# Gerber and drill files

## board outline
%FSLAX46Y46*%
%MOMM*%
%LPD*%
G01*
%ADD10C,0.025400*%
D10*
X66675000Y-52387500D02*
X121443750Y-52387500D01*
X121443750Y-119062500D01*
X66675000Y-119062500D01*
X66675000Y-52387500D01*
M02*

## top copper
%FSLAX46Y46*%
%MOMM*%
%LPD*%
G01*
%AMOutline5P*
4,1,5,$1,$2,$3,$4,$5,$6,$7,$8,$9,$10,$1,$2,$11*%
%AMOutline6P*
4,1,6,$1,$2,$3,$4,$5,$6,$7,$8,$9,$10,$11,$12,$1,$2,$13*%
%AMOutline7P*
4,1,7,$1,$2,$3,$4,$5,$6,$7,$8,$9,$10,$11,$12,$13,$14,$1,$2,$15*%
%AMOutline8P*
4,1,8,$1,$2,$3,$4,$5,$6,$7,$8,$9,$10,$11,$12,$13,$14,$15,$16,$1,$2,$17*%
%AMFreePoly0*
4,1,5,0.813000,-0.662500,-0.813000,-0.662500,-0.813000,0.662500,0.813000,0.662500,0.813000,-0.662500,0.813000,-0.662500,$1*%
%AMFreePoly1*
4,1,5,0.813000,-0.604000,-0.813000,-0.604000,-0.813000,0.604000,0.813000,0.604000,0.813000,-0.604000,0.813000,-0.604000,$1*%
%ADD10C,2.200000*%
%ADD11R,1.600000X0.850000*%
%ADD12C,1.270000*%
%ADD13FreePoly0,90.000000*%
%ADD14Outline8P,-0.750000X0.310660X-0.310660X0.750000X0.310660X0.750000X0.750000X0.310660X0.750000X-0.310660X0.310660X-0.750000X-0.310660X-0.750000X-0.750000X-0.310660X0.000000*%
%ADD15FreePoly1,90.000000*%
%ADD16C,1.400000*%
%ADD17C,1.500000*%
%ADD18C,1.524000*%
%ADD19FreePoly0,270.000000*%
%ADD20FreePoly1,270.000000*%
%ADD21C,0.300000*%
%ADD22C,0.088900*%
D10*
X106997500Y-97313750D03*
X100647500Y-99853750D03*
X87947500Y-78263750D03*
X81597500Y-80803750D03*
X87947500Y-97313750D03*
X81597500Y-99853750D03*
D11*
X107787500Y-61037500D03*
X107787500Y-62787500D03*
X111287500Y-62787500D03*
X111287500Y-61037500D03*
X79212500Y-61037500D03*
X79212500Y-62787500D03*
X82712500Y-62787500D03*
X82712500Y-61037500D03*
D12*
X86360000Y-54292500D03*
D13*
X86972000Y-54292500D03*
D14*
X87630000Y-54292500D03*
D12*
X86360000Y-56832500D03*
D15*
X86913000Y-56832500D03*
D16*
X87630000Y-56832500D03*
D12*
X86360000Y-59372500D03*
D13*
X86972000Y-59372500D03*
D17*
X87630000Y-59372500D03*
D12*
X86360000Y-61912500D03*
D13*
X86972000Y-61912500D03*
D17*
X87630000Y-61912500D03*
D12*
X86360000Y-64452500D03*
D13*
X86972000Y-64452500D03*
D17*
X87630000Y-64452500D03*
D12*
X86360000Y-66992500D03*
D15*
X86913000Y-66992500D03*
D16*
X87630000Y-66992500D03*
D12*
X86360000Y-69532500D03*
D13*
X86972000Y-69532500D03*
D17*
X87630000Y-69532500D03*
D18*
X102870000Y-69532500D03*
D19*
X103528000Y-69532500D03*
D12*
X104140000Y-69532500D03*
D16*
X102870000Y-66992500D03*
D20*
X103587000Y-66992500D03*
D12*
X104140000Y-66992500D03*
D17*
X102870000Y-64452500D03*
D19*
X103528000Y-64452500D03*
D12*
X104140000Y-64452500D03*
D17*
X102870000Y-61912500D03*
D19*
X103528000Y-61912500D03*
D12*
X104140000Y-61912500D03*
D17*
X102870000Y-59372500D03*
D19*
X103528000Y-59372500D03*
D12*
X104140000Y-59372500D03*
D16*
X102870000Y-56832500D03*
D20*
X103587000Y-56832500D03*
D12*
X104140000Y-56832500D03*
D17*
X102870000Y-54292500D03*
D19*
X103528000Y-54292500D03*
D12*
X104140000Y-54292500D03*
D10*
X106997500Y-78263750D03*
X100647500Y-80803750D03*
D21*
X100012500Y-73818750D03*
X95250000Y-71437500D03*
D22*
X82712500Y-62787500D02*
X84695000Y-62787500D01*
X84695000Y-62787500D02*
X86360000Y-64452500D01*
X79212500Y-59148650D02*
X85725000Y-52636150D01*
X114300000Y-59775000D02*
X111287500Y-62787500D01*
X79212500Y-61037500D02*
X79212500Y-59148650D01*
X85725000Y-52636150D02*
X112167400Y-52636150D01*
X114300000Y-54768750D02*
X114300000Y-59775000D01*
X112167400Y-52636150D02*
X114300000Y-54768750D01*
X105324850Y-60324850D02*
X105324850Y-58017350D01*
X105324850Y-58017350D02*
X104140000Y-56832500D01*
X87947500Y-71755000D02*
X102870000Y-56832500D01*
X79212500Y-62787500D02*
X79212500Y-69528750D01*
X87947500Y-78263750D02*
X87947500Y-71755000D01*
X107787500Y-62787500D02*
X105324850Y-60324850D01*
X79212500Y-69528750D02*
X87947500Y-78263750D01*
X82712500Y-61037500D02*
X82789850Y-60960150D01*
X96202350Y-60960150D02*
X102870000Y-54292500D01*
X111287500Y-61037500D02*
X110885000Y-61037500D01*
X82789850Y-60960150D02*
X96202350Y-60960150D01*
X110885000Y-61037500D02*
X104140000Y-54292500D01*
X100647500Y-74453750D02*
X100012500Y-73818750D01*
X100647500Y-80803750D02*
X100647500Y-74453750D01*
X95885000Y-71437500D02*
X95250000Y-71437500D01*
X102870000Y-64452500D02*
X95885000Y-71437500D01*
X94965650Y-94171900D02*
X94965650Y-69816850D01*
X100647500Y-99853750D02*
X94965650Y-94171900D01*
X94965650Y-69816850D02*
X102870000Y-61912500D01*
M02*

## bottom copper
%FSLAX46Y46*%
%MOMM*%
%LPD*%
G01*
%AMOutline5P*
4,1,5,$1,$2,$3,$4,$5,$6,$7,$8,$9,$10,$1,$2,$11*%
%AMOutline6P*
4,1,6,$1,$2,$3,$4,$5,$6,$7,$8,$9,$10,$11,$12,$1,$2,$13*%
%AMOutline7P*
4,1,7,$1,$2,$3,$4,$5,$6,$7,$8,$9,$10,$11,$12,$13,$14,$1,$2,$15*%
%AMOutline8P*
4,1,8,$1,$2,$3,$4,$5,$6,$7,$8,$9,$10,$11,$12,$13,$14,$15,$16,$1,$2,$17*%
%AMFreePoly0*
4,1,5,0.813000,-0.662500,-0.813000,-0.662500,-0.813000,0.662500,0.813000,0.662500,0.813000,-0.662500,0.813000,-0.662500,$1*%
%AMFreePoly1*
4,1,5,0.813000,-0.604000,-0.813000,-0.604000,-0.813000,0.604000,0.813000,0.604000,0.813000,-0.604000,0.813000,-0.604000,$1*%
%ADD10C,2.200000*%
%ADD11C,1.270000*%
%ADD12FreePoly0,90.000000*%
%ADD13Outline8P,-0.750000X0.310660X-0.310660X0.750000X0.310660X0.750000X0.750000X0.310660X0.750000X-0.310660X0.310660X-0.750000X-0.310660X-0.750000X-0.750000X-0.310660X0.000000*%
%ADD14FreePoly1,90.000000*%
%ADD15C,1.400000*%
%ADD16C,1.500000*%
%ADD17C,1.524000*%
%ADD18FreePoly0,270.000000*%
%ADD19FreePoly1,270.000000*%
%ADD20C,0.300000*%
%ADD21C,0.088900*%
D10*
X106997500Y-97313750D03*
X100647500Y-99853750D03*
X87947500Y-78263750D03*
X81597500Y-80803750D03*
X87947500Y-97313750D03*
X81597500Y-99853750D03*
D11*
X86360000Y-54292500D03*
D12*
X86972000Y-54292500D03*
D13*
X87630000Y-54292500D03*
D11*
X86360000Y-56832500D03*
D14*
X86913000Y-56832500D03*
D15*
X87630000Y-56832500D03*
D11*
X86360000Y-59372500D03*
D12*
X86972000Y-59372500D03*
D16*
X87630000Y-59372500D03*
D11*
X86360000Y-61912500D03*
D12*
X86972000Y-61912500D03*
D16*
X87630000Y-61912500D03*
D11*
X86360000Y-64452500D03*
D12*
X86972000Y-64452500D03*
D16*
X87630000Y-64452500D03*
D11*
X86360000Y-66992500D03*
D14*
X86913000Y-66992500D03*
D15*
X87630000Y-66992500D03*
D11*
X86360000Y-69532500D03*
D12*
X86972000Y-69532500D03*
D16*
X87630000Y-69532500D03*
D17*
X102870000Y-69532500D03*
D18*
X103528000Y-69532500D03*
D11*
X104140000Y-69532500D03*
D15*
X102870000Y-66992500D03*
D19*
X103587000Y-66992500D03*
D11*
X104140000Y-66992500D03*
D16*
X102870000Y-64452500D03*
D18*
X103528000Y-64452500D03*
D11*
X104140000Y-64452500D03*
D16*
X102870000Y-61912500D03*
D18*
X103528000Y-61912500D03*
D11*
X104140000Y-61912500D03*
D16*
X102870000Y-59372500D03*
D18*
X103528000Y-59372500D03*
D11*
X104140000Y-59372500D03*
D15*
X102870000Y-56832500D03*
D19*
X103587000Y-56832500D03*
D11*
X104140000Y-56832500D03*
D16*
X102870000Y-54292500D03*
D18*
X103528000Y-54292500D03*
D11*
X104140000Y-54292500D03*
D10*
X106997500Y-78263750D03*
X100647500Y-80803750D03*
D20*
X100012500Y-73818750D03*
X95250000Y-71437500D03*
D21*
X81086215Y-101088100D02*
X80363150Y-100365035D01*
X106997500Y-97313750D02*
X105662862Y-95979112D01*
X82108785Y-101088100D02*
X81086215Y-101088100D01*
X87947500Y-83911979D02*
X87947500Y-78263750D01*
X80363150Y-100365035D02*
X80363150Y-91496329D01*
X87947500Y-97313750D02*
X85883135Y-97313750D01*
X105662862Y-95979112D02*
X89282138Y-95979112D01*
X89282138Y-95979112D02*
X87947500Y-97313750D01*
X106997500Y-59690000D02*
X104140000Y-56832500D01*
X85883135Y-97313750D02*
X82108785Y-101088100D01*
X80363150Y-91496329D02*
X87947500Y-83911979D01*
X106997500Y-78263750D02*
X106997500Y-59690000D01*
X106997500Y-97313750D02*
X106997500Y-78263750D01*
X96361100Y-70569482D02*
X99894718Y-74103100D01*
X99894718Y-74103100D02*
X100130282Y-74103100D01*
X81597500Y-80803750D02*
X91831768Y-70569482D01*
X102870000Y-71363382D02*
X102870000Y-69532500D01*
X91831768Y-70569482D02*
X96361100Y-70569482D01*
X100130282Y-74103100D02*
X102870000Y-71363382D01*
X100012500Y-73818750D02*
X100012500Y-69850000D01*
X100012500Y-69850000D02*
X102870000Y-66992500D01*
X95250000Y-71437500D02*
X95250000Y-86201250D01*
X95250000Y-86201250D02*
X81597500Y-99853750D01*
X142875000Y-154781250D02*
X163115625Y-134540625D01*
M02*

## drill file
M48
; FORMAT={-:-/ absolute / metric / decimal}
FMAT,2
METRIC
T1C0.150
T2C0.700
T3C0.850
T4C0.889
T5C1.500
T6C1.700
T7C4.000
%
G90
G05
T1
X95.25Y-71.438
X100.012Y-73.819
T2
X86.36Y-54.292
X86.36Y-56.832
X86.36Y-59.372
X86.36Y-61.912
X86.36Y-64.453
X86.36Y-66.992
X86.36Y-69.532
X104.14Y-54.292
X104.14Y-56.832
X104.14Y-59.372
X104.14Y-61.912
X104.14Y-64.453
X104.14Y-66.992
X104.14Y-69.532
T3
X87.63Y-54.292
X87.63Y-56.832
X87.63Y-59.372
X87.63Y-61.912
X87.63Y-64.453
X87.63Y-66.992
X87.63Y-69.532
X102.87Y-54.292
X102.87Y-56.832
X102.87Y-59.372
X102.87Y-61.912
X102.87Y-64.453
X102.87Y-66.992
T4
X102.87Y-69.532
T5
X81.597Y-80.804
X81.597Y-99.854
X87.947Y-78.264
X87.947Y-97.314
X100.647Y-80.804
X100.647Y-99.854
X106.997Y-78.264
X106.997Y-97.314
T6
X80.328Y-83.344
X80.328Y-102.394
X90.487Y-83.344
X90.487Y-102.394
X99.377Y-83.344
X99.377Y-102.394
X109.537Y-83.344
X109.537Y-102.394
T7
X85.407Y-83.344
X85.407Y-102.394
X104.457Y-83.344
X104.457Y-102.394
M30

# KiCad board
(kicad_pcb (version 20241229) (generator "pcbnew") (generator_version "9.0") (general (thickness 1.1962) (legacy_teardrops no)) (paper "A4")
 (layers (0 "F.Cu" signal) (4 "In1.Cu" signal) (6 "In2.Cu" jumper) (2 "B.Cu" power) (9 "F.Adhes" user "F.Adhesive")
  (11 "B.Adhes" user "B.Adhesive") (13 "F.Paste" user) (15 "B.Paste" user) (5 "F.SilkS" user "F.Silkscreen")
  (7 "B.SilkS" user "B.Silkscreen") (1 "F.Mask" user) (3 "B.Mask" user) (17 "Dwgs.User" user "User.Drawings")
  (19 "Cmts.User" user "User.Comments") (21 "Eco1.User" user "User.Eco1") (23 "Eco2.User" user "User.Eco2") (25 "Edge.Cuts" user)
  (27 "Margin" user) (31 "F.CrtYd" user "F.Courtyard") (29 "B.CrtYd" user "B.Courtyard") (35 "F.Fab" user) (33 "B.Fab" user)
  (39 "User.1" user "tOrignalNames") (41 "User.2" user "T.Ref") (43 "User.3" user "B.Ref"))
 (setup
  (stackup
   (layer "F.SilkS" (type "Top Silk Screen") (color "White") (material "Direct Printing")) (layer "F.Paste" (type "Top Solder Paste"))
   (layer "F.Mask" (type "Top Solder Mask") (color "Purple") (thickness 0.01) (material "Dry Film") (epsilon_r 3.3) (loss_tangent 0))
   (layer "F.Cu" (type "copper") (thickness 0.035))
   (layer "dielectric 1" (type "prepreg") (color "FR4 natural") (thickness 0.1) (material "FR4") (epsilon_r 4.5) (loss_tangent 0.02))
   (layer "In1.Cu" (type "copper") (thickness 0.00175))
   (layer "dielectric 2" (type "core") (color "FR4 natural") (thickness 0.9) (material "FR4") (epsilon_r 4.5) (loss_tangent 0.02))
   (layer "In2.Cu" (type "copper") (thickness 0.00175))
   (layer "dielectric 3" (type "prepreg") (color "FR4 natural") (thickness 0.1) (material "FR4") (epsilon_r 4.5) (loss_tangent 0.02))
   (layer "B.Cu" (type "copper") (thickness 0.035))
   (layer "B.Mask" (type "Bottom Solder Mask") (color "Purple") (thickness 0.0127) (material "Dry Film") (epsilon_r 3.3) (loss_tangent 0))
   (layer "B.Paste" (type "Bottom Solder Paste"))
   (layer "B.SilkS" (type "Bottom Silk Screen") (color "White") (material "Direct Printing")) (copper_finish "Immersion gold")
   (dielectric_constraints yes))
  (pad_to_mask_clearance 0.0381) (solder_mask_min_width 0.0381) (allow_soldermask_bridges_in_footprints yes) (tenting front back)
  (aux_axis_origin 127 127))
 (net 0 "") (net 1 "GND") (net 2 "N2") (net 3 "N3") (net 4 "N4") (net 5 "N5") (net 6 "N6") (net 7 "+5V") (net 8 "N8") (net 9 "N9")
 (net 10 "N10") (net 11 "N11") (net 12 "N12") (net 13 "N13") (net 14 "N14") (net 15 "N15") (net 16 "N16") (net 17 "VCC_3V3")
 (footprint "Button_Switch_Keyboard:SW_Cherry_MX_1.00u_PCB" (layer "F.Cu") (at 106.9975 97.31375)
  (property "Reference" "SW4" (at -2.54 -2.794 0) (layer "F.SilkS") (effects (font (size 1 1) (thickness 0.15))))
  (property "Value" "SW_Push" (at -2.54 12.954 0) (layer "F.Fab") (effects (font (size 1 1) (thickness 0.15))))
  (pad "" np_thru_hole circle (at -7.62 5.08) (size 1.7 1.7) (drill 1.7) (layers "*.Cu" "*.Mask"))
  (pad "" np_thru_hole circle (at -2.54 5.08) (size 4 4) (drill 4) (layers "*.Cu" "*.Mask"))
  (pad "" np_thru_hole circle (at 2.54 5.08) (size 1.7 1.7) (drill 1.7) (layers "*.Cu" "*.Mask"))
  (pad "1" thru_hole circle (at 0 0) (size 2.2 2.2) (drill 1.5) (layers "*.Cu" "*.Mask") (remove_unused_layers no) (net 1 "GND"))
  (pad "2" thru_hole circle (at -6.35 2.54) (size 2.2 2.2) (drill 1.5) (layers "*.Cu" "*.Mask") (remove_unused_layers no) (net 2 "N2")))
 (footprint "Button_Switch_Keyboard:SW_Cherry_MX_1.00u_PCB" (layer "F.Cu") (at 87.9475 78.26375)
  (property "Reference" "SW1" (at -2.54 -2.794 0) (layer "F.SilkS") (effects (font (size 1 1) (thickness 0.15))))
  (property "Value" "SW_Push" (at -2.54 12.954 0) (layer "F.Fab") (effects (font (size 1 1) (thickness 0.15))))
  (pad "" np_thru_hole circle (at -7.62 5.08) (size 1.7 1.7) (drill 1.7) (layers "*.Cu" "*.Mask"))
  (pad "" np_thru_hole circle (at -2.54 5.08) (size 4 4) (drill 4) (layers "*.Cu" "*.Mask"))
  (pad "" np_thru_hole circle (at 2.54 5.08) (size 1.7 1.7) (drill 1.7) (layers "*.Cu" "*.Mask"))
  (pad "1" thru_hole circle (at 0 0) (size 2.2 2.2) (drill 1.5) (layers "*.Cu" "*.Mask") (remove_unused_layers no) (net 1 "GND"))
  (pad "2" thru_hole circle (at -6.35 2.54) (size 2.2 2.2) (drill 1.5) (layers "*.Cu" "*.Mask") (remove_unused_layers no) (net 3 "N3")))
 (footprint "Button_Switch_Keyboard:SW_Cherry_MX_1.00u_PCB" (layer "F.Cu") (at 87.9475 97.31375)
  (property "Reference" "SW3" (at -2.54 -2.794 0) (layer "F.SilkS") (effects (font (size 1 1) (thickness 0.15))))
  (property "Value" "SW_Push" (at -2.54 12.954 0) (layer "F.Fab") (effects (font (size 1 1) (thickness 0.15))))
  (pad "" np_thru_hole circle (at -7.62 5.08) (size 1.7 1.7) (drill 1.7) (layers "*.Cu" "*.Mask"))
  (pad "" np_thru_hole circle (at -2.54 5.08) (size 4 4) (drill 4) (layers "*.Cu" "*.Mask"))
  (pad "" np_thru_hole circle (at 2.54 5.08) (size 1.7 1.7) (drill 1.7) (layers "*.Cu" "*.Mask"))
  (pad "1" thru_hole circle (at 0 0) (size 2.2 2.2) (drill 1.5) (layers "*.Cu" "*.Mask") (remove_unused_layers no) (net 1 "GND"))
  (pad "2" thru_hole circle (at -6.35 2.54) (size 2.2 2.2) (drill 1.5) (layers "*.Cu" "*.Mask") (remove_unused_layers no) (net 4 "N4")))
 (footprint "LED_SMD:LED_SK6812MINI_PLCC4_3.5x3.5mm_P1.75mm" (layer "F.Cu") (at 109.5375 61.9125)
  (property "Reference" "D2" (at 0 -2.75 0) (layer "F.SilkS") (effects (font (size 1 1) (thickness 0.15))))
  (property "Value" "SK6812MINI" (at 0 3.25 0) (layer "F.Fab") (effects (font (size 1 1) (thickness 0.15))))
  (pad "1" smd rect (at -1.75 -0.875) (size 1.6 0.85) (layers "F.Cu" "F.Mask" "F.Paste") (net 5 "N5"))
  (pad "2" smd rect (at -1.75 0.875) (size 1.6 0.85) (layers "F.Cu" "F.Mask" "F.Paste") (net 1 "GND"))
  (pad "3" smd rect (at 1.75 0.875) (size 1.6 0.85) (layers "F.Cu" "F.Mask" "F.Paste") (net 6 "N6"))
  (pad "4" smd rect (at 1.75 -0.875) (size 1.6 0.85) (layers "F.Cu" "F.Mask" "F.Paste") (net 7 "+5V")))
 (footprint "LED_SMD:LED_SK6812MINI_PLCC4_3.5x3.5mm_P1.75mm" (layer "F.Cu") (at 80.9625 61.9125)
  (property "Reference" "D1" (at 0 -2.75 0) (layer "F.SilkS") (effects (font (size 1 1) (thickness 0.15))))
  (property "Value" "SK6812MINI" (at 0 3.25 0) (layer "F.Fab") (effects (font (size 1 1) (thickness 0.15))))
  (pad "1" smd rect (at -1.75 -0.875) (size 1.6 0.85) (layers "F.Cu" "F.Mask" "F.Paste") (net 6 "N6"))
  (pad "2" smd rect (at -1.75 0.875) (size 1.6 0.85) (layers "F.Cu" "F.Mask" "F.Paste") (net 1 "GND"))
  (pad "3" smd rect (at 1.75 0.875) (size 1.6 0.85) (layers "F.Cu" "F.Mask" "F.Paste") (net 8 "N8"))
  (pad "4" smd rect (at 1.75 -0.875) (size 1.6 0.85) (layers "F.Cu" "F.Mask" "F.Paste") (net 7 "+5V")))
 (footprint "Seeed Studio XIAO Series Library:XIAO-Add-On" (layer "F.Cu") (at 95.25 61.9125)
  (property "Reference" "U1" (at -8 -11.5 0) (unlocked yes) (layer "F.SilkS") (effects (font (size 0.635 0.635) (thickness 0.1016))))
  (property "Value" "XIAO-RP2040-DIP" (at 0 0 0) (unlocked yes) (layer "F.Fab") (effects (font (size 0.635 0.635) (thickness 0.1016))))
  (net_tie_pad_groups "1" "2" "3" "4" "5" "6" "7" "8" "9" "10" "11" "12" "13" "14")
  (pad "1" thru_hole circle (at -8.89 -7.62 270) (size 1.27 1.27) (drill 0.7) (layers "*.Cu" "*.Mask") (remove_unused_layers no)
   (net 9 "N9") (solder_mask_margin 0.0254))
  (pad "1" smd custom (at -8.278 -7.62 90) (size 1.626 1.325) (layers "F.Cu" "F.Mask" "F.Paste") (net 9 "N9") (solder_mask_margin 0.05)
   (options (clearance outline) (anchor rect)) (primitives))
  (pad "1" smd custom (at -8.278 -7.62 90) (size 1.626 1.325) (layers "B.Cu" "B.Mask" "B.Paste") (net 9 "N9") (solder_mask_margin 0.05)
   (options (clearance outline) (anchor rect)) (primitives))
  (pad "1" thru_hole roundrect (at -7.62 -7.62) (size 1.5 1.5) (drill 0.85) (layers "*.Cu" "*.Mask") (remove_unused_layers no)
   (roundrect_rratio 0.25) (chamfer_ratio 0.2928932188) (chamfer top_left top_right bottom_left bottom_right) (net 9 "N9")
   (solder_mask_margin 0.0254) (thermal_bridge_angle 45))
  (pad "2" thru_hole circle (at -8.89 -5.08 270) (size 1.27 1.27) (drill 0.7) (layers "*.Cu" "*.Mask") (remove_unused_layers no)
   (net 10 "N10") (solder_mask_margin 0.0254))
  (pad "2" smd custom (at -8.337 -5.08 90) (size 1.626 1.208) (layers "F.Cu" "F.Mask" "F.Paste") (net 10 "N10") (solder_mask_margin 0.05)
   (options (clearance outline) (anchor rect)) (primitives))
  (pad "2" smd custom (at -8.337 -5.08 90) (size 1.626 1.208) (layers "B.Cu" "B.Mask" "B.Paste") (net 10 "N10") (solder_mask_margin 0.05)
   (options (clearance outline) (anchor rect)) (primitives))
  (pad "2" thru_hole circle (at -7.62 -5.08) (size 1.4 1.4) (drill 0.85) (layers "*.Cu") (remove_unused_layers no) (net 10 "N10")
   (solder_mask_margin 0.0254))
  (pad "3" thru_hole circle (at -8.89 -2.54 270) (size 1.27 1.27) (drill 0.7) (layers "*.Cu" "*.Mask") (remove_unused_layers no)
   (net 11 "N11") (solder_mask_margin 0.0254))
  (pad "3" smd custom (at -8.278 -2.54 90) (size 1.626 1.325) (layers "F.Cu" "F.Mask" "F.Paste") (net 11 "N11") (solder_mask_margin 0.05)
   (options (clearance outline) (anchor rect)) (primitives))
  (pad "3" smd custom (at -8.278 -2.54 90) (size 1.626 1.325) (layers "B.Cu" "B.Mask" "B.Paste") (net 11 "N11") (solder_mask_margin 0.05)
   (options (clearance outline) (anchor rect)) (primitives))
  (pad "3" thru_hole circle (at -7.62 -2.54) (size 1.5 1.5) (drill 0.85) (layers "*.Cu" "*.Mask") (remove_unused_layers no) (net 11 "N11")
   (solder_mask_margin 0.0254))
  (pad "4" thru_hole circle (at -8.89 0 270) (size 1.27 1.27) (drill 0.7) (layers "*.Cu" "*.Mask") (remove_unused_layers no) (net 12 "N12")
   (solder_mask_margin 0.0254))
  (pad "4" smd custom (at -8.278 0 90) (size 1.626 1.325) (layers "F.Cu" "F.Mask" "F.Paste") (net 12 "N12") (solder_mask_margin 0.05)
   (options (clearance outline) (anchor rect)) (primitives))
  (pad "4" smd custom (at -8.278 0 90) (size 1.626 1.325) (layers "B.Cu" "B.Mask" "B.Paste") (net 12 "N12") (solder_mask_margin 0.05)
   (options (clearance outline) (anchor rect)) (primitives))
  (pad "4" thru_hole circle (at -7.62 0) (size 1.5 1.5) (drill 0.85) (layers "*.Cu" "*.Mask") (remove_unused_layers no) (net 12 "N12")
   (solder_mask_margin 0.0254))
  (pad "5" thru_hole circle (at -8.89 2.54 270) (size 1.27 1.27) (drill 0.7) (layers "*.Cu" "*.Mask") (remove_unused_layers no) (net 8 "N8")
   (solder_mask_margin 0.0254))
  (pad "5" smd custom (at -8.278 2.54 90) (size 1.626 1.325) (layers "F.Cu" "F.Mask" "F.Paste") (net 8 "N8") (solder_mask_margin 0.05)
   (options (clearance outline) (anchor rect)) (primitives))
  (pad "5" smd custom (at -8.278 2.54 90) (size 1.626 1.325) (layers "B.Cu" "B.Mask" "B.Paste") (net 8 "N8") (solder_mask_margin 0.05)
   (options (clearance outline) (anchor rect)) (primitives))
  (pad "5" thru_hole circle (at -7.62 2.54) (size 1.5 1.5) (drill 0.85) (layers "*.Cu" "*.Mask") (remove_unused_layers no) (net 8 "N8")
   (solder_mask_margin 0.0254))
  (pad "6" thru_hole circle (at -8.89 5.08 270) (size 1.27 1.27) (drill 0.7) (layers "*.Cu" "*.Mask") (remove_unused_layers no)
   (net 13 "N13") (solder_mask_margin 0.0254))
  (pad "6" smd custom (at -8.337 5.08 90) (size 1.626 1.208) (layers "F.Cu" "F.Mask" "F.Paste") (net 13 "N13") (solder_mask_margin 0.05)
   (options (clearance outline) (anchor rect)) (primitives))
  (pad "6" smd custom (at -8.337 5.08 90) (size 1.626 1.208) (layers "B.Cu" "B.Mask" "B.Paste") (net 13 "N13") (solder_mask_margin 0.05)
   (options (clearance outline) (anchor rect)) (primitives))
  (pad "6" thru_hole circle (at -7.62 5.08) (size 1.4 1.4) (drill 0.85) (layers "*.Cu") (remove_unused_layers no) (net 13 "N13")
   (solder_mask_margin 0.0254))
  (pad "7" thru_hole circle (at -8.89 7.62 270) (size 1.27 1.27) (drill 0.7) (layers "*.Cu" "*.Mask") (remove_unused_layers no)
   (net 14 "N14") (solder_mask_margin 0.0254))
  (pad "7" smd custom (at -8.278 7.62 90) (size 1.626 1.325) (layers "F.Cu" "F.Mask" "F.Paste") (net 14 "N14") (solder_mask_margin 0.05)
   (options (clearance outline) (anchor rect)) (primitives))
  (pad "7" smd custom (at -8.278 7.62 90) (size 1.626 1.325) (layers "B.Cu" "B.Mask" "B.Paste") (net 14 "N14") (solder_mask_margin 0.05)
   (options (clearance outline) (anchor rect)) (primitives))
  (pad "7" thru_hole circle (at -7.62 7.62) (size 1.5 1.5) (drill 0.85) (layers "*.Cu" "*.Mask") (remove_unused_layers no) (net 14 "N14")
   (solder_mask_margin 0.0254))
  (pad "8" thru_hole circle (at 7.62 7.62) (size 1.524 1.524) (drill 0.889) (layers "*.Cu" "*.Mask") (remove_unused_layers no) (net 3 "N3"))
  (pad "8" smd custom (at 8.278 7.62 270) (size 1.626 1.325) (layers "F.Cu" "F.Mask" "F.Paste") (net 3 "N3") (solder_mask_margin 0.05)
   (options (clearance outline) (anchor rect)) (primitives))
  (pad "8" smd custom (at 8.278 7.62 270) (size 1.626 1.325) (layers "B.Cu" "B.Mask" "B.Paste") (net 3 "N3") (solder_mask_margin 0.05)
   (options (clearance outline) (anchor rect)) (primitives))
  (pad "8" thru_hole circle (at 8.89 7.62 90) (size 1.27 1.27) (drill 0.7) (layers "*.Cu" "*.Mask") (remove_unused_layers no) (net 3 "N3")
   (solder_mask_margin 0.0254))
  (pad "9" thru_hole circle (at 7.62 5.08 180) (size 1.4 1.4) (drill 0.85) (layers "*.Cu") (remove_unused_layers no) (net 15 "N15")
   (solder_mask_margin 0.0254))
  (pad "9" smd custom (at 8.337 5.08 270) (size 1.626 1.208) (layers "F.Cu" "F.Mask" "F.Paste") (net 15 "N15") (solder_mask_margin 0.05)
   (options (clearance outline) (anchor rect)) (primitives))
  (pad "9" smd custom (at 8.337 5.08 270) (size 1.626 1.208) (layers "B.Cu" "B.Mask" "B.Paste") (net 15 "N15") (solder_mask_margin 0.05)
   (options (clearance outline) (anchor rect)) (primitives))
  (pad "9" thru_hole circle (at 8.89 5.08 90) (size 1.27 1.27) (drill 0.7) (layers "*.Cu" "*.Mask") (remove_unused_layers no) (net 15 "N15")
   (solder_mask_margin 0.0254))
  (pad "10" thru_hole circle (at 7.62 2.54 180) (size 1.5 1.5) (drill 0.85) (layers "*.Cu" "*.Mask") (remove_unused_layers no) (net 4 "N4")
   (solder_mask_margin 0.0254))
  (pad "10" smd custom (at 8.278 2.54 270) (size 1.626 1.325) (layers "F.Cu" "F.Mask" "F.Paste") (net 4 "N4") (solder_mask_margin 0.05)
   (options (clearance outline) (anchor rect)) (primitives))
  (pad "10" smd custom (at 8.278 2.54 270) (size 1.626 1.325) (layers "B.Cu" "B.Mask" "B.Paste") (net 4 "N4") (solder_mask_margin 0.05)
   (options (clearance outline) (anchor rect)) (primitives))
  (pad "10" thru_hole circle (at 8.89 2.54 90) (size 1.27 1.27) (drill 0.7) (layers "*.Cu" "*.Mask") (remove_unused_layers no) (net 4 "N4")
   (solder_mask_margin 0.0254))
  (pad "11" thru_hole circle (at 7.62 0 180) (size 1.5 1.5) (drill 0.85) (layers "*.Cu" "*.Mask") (remove_unused_layers no) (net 2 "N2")
   (solder_mask_margin 0.0254))
  (pad "11" smd custom (at 8.278 0 270) (size 1.626 1.325) (layers "F.Cu" "F.Mask" "F.Paste") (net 2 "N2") (solder_mask_margin 0.05)
   (options (clearance outline) (anchor rect)) (primitives))
  (pad "11" smd custom (at 8.278 0 270) (size 1.626 1.325) (layers "B.Cu" "B.Mask" "B.Paste") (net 2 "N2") (solder_mask_margin 0.05)
   (options (clearance outline) (anchor rect)) (primitives))
  (pad "11" thru_hole circle (at 8.89 0 90) (size 1.27 1.27) (drill 0.7) (layers "*.Cu" "*.Mask") (remove_unused_layers no) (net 2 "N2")
   (solder_mask_margin 0.0254))
  (pad "12" thru_hole circle (at 7.62 -2.54 180) (size 1.5 1.5) (drill 0.85) (layers "*.Cu" "*.Mask") (remove_unused_layers no)
   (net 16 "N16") (solder_mask_margin 0.0254))
  (pad "12" smd custom (at 8.278 -2.54 270) (size 1.626 1.325) (layers "F.Cu" "F.Mask" "F.Paste") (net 16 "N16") (solder_mask_margin 0.05)
   (options (clearance outline) (anchor rect)) (primitives))
  (pad "12" smd custom (at 8.278 -2.54 270) (size 1.626 1.325) (layers "B.Cu" "B.Mask" "B.Paste") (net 16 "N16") (solder_mask_margin 0.05)
   (options (clearance outline) (anchor rect)) (primitives))
  (pad "12" thru_hole circle (at 8.89 -2.54 90) (size 1.27 1.27) (drill 0.7) (layers "*.Cu" "*.Mask") (remove_unused_layers no)
   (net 16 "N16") (solder_mask_margin 0.0254))
  (pad "13" thru_hole circle (at 7.62 -5.08 180) (size 1.4 1.4) (drill 0.85) (layers "*.Cu") (remove_unused_layers no) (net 1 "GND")
   (solder_mask_margin 0.0254))
  (pad "13" smd custom (at 8.337 -5.08 270) (size 1.626 1.208) (layers "F.Cu" "F.Mask" "F.Paste") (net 1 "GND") (solder_mask_margin 0.05)
   (options (clearance outline) (anchor rect)) (primitives))
  (pad "13" smd custom (at 8.337 -5.08 270) (size 1.626 1.208) (layers "B.Cu" "B.Mask" "B.Paste") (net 1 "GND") (solder_mask_margin 0.05)
   (options (clearance outline) (anchor rect)) (primitives))
  (pad "13" thru_hole circle (at 8.89 -5.08 90) (size 1.27 1.27) (drill 0.7) (layers "*.Cu" "*.Mask") (remove_unused_layers no)
   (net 1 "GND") (solder_mask_margin 0.0254))
  (pad "14" thru_hole circle (at 7.62 -7.62 180) (size 1.5 1.5) (drill 0.85) (layers "*.Cu" "*.Mask") (remove_unused_layers no)
   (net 7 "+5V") (solder_mask_margin 0.0254))
  (pad "14" smd custom (at 8.278 -7.62 270) (size 1.626 1.325) (layers "F.Cu" "F.Mask" "F.Paste") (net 7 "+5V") (solder_mask_margin 0.05)
   (options (clearance outline) (anchor rect)) (primitives))
  (pad "14" smd custom (at 8.278 -7.62 270) (size 1.626 1.325) (layers "B.Cu" "B.Mask" "B.Paste") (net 7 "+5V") (solder_mask_margin 0.05)
   (options (clearance outline) (anchor rect)) (primitives))
  (pad "14" thru_hole circle (at 8.89 -7.62 90) (size 1.27 1.27) (drill 0.7) (layers "*.Cu" "*.Mask") (remove_unused_layers no)
   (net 7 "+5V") (solder_mask_margin 0.0254)))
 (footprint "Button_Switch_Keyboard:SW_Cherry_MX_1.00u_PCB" (layer "F.Cu") (at 106.9975 78.26375)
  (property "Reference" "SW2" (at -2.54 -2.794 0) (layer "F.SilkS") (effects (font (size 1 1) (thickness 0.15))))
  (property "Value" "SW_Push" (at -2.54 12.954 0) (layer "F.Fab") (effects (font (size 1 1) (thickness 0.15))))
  (pad "" np_thru_hole circle (at -7.62 5.08) (size 1.7 1.7) (drill 1.7) (layers "*.Cu" "*.Mask"))
  (pad "" np_thru_hole circle (at -2.54 5.08) (size 4 4) (drill 4) (layers "*.Cu" "*.Mask"))
  (pad "" np_thru_hole circle (at 2.54 5.08) (size 1.7 1.7) (drill 1.7) (layers "*.Cu" "*.Mask"))
  (pad "1" thru_hole circle (at 0 0) (size 2.2 2.2) (drill 1.5) (layers "*.Cu" "*.Mask") (remove_unused_layers no) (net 1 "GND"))
  (pad "2" thru_hole circle (at -6.35 2.54) (size 2.2 2.2) (drill 1.5) (layers "*.Cu" "*.Mask") (remove_unused_layers no) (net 15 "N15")))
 (gr_rect (start 66.675 52.3875) (end 121.44375 119.0625) (stroke (width 0.0254) (type default)) (fill no) (layer "Edge.Cuts"))
 (segment (start 82.7125 62.7875) (end 84.695 62.7875) (width 0.0889) (layer "F.Cu") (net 8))
 (segment (start 84.695 62.7875) (end 86.36 64.4525) (width 0.0889) (layer "F.Cu") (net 8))
 (segment (start 79.2125 59.14865) (end 85.725 52.63615) (width 0.0889) (layer "F.Cu") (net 6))
 (segment (start 114.3 59.775) (end 111.2875 62.7875) (width 0.0889) (layer "F.Cu") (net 6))
 (segment (start 79.2125 61.0375) (end 79.2125 59.14865) (width 0.0889) (layer "F.Cu") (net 6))
 (segment (start 85.725 52.63615) (end 112.1674 52.63615) (width 0.0889) (layer "F.Cu") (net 6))
 (segment (start 114.3 54.76875) (end 114.3 59.775) (width 0.0889) (layer "F.Cu") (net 6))
 (segment (start 112.1674 52.63615) (end 114.3 54.76875) (width 0.0889) (layer "F.Cu") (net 6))
 (segment (start 105.32485 60.32485) (end 105.32485 58.01735) (width 0.0889) (layer "F.Cu") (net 1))
 (segment (start 105.32485 58.01735) (end 104.14 56.8325) (width 0.0889) (layer "F.Cu") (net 1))
 (segment (start 87.9475 71.755) (end 102.87 56.8325) (width 0.0889) (layer "F.Cu") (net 1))
 (segment (start 79.2125 62.7875) (end 79.2125 69.52875) (width 0.0889) (layer "F.Cu") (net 1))
 (segment (start 87.9475 78.26375) (end 87.9475 71.755) (width 0.0889) (layer "F.Cu") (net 1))
 (segment (start 107.7875 62.7875) (end 105.32485 60.32485) (width 0.0889) (layer "F.Cu") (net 1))
 (segment (start 79.2125 69.52875) (end 87.9475 78.26375) (width 0.0889) (layer "F.Cu") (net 1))
 (segment (start 81.086215 101.0881) (end 80.36315 100.365035) (width 0.0889) (layer "B.Cu") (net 1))
 (segment (start 106.9975 97.31375) (end 105.662862 95.979112) (width 0.0889) (layer "B.Cu") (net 1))
 (segment (start 82.108785 101.0881) (end 81.086215 101.0881) (width 0.0889) (layer "B.Cu") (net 1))
 (segment (start 87.9475 83.911979) (end 87.9475 78.26375) (width 0.0889) (layer "B.Cu") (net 1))
 (segment (start 80.36315 100.365035) (end 80.36315 91.496329) (width 0.0889) (layer "B.Cu") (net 1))
 (segment (start 87.9475 97.31375) (end 85.883135 97.31375) (width 0.0889) (layer "B.Cu") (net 1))
 (segment (start 105.662862 95.979112) (end 89.282138 95.979112) (width 0.0889) (layer "B.Cu") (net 1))
 (segment (start 89.282138 95.979112) (end 87.9475 97.31375) (width 0.0889) (layer "B.Cu") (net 1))
 (segment (start 106.9975 59.69) (end 104.14 56.8325) (width 0.0889) (layer "B.Cu") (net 1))
 (segment (start 85.883135 97.31375) (end 82.108785 101.0881) (width 0.0889) (layer "B.Cu") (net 1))
 (segment (start 80.36315 91.496329) (end 87.9475 83.911979) (width 0.0889) (layer "B.Cu") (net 1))
 (segment (start 106.9975 78.26375) (end 106.9975 59.69) (width 0.0889) (layer "B.Cu") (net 1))
 (segment (start 106.9975 97.31375) (end 106.9975 78.26375) (width 0.0889) (layer "B.Cu") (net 1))
 (segment (start 82.7125 61.0375) (end 82.78985 60.96015) (width 0.0889) (layer "F.Cu") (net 7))
 (segment (start 96.20235 60.96015) (end 102.87 54.2925) (width 0.0889) (layer "F.Cu") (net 7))
 (segment (start 111.2875 61.0375) (end 110.885 61.0375) (width 0.0889) (layer "F.Cu") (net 7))
 (segment (start 82.78985 60.96015) (end 96.20235 60.96015) (width 0.0889) (layer "F.Cu") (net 7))
 (segment (start 110.885 61.0375) (end 104.14 54.2925) (width 0.0889) (layer "F.Cu") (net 7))
 (segment (start 96.3611 70.569482) (end 99.894718 74.1031) (width 0.0889) (layer "B.Cu") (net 3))
 (segment (start 99.894718 74.1031) (end 100.130282 74.1031) (width 0.0889) (layer "B.Cu") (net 3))
 (segment (start 81.5975 80.80375) (end 91.831768 70.569482) (width 0.0889) (layer "B.Cu") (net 3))
 (segment (start 102.87 71.363382) (end 102.87 69.5325) (width 0.0889) (layer "B.Cu") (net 3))
 (segment (start 91.831768 70.569482) (end 96.3611 70.569482) (width 0.0889) (layer "B.Cu") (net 3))
 (segment (start 100.130282 74.1031) (end 102.87 71.363382) (width 0.0889) (layer "B.Cu") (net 3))
 (segment (start 100.6475 74.45375) (end 100.0125 73.81875) (width 0.0889) (layer "F.Cu") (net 15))
 (segment (start 100.6475 80.80375) (end 100.6475 74.45375) (width 0.0889) (layer "F.Cu") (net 15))
 (via (at 100.0125 73.81875) (size 0.3) (drill 0.15) (layers "F.Cu" "B.Cu") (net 15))
 (segment (start 100.0125 73.81875) (end 100.0125 69.85) (width 0.0889) (layer "B.Cu") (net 15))
 (segment (start 100.0125 69.85) (end 102.87 66.9925) (width 0.0889) (layer "B.Cu") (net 15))
 (segment (start 95.885 71.4375) (end 95.25 71.4375) (width 0.0889) (layer "F.Cu") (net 4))
 (segment (start 102.87 64.4525) (end 95.885 71.4375) (width 0.0889) (layer "F.Cu") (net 4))
 (via (at 95.25 71.4375) (size 0.3) (drill 0.15) (layers "F.Cu" "B.Cu") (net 4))
 (segment (start 95.25 71.4375) (end 95.25 86.20125) (width 0.0889) (layer "B.Cu") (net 4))
 (segment (start 95.25 86.20125) (end 81.5975 99.85375) (width 0.0889) (layer "B.Cu") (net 4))
 (segment (start 94.96565 94.1719) (end 94.96565 69.81685) (width 0.0889) (layer "F.Cu") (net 2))
 (segment (start 100.6475 99.85375) (end 94.96565 94.1719) (width 0.0889) (layer "F.Cu") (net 2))
 (segment (start 94.96565 69.81685) (end 102.87 61.9125) (width 0.0889) (layer "F.Cu") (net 2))
 (segment (start 142.875 154.78125) (end 163.115625 134.540625) (width 0.0889) (locked yes) (layer "B.Cu") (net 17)))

